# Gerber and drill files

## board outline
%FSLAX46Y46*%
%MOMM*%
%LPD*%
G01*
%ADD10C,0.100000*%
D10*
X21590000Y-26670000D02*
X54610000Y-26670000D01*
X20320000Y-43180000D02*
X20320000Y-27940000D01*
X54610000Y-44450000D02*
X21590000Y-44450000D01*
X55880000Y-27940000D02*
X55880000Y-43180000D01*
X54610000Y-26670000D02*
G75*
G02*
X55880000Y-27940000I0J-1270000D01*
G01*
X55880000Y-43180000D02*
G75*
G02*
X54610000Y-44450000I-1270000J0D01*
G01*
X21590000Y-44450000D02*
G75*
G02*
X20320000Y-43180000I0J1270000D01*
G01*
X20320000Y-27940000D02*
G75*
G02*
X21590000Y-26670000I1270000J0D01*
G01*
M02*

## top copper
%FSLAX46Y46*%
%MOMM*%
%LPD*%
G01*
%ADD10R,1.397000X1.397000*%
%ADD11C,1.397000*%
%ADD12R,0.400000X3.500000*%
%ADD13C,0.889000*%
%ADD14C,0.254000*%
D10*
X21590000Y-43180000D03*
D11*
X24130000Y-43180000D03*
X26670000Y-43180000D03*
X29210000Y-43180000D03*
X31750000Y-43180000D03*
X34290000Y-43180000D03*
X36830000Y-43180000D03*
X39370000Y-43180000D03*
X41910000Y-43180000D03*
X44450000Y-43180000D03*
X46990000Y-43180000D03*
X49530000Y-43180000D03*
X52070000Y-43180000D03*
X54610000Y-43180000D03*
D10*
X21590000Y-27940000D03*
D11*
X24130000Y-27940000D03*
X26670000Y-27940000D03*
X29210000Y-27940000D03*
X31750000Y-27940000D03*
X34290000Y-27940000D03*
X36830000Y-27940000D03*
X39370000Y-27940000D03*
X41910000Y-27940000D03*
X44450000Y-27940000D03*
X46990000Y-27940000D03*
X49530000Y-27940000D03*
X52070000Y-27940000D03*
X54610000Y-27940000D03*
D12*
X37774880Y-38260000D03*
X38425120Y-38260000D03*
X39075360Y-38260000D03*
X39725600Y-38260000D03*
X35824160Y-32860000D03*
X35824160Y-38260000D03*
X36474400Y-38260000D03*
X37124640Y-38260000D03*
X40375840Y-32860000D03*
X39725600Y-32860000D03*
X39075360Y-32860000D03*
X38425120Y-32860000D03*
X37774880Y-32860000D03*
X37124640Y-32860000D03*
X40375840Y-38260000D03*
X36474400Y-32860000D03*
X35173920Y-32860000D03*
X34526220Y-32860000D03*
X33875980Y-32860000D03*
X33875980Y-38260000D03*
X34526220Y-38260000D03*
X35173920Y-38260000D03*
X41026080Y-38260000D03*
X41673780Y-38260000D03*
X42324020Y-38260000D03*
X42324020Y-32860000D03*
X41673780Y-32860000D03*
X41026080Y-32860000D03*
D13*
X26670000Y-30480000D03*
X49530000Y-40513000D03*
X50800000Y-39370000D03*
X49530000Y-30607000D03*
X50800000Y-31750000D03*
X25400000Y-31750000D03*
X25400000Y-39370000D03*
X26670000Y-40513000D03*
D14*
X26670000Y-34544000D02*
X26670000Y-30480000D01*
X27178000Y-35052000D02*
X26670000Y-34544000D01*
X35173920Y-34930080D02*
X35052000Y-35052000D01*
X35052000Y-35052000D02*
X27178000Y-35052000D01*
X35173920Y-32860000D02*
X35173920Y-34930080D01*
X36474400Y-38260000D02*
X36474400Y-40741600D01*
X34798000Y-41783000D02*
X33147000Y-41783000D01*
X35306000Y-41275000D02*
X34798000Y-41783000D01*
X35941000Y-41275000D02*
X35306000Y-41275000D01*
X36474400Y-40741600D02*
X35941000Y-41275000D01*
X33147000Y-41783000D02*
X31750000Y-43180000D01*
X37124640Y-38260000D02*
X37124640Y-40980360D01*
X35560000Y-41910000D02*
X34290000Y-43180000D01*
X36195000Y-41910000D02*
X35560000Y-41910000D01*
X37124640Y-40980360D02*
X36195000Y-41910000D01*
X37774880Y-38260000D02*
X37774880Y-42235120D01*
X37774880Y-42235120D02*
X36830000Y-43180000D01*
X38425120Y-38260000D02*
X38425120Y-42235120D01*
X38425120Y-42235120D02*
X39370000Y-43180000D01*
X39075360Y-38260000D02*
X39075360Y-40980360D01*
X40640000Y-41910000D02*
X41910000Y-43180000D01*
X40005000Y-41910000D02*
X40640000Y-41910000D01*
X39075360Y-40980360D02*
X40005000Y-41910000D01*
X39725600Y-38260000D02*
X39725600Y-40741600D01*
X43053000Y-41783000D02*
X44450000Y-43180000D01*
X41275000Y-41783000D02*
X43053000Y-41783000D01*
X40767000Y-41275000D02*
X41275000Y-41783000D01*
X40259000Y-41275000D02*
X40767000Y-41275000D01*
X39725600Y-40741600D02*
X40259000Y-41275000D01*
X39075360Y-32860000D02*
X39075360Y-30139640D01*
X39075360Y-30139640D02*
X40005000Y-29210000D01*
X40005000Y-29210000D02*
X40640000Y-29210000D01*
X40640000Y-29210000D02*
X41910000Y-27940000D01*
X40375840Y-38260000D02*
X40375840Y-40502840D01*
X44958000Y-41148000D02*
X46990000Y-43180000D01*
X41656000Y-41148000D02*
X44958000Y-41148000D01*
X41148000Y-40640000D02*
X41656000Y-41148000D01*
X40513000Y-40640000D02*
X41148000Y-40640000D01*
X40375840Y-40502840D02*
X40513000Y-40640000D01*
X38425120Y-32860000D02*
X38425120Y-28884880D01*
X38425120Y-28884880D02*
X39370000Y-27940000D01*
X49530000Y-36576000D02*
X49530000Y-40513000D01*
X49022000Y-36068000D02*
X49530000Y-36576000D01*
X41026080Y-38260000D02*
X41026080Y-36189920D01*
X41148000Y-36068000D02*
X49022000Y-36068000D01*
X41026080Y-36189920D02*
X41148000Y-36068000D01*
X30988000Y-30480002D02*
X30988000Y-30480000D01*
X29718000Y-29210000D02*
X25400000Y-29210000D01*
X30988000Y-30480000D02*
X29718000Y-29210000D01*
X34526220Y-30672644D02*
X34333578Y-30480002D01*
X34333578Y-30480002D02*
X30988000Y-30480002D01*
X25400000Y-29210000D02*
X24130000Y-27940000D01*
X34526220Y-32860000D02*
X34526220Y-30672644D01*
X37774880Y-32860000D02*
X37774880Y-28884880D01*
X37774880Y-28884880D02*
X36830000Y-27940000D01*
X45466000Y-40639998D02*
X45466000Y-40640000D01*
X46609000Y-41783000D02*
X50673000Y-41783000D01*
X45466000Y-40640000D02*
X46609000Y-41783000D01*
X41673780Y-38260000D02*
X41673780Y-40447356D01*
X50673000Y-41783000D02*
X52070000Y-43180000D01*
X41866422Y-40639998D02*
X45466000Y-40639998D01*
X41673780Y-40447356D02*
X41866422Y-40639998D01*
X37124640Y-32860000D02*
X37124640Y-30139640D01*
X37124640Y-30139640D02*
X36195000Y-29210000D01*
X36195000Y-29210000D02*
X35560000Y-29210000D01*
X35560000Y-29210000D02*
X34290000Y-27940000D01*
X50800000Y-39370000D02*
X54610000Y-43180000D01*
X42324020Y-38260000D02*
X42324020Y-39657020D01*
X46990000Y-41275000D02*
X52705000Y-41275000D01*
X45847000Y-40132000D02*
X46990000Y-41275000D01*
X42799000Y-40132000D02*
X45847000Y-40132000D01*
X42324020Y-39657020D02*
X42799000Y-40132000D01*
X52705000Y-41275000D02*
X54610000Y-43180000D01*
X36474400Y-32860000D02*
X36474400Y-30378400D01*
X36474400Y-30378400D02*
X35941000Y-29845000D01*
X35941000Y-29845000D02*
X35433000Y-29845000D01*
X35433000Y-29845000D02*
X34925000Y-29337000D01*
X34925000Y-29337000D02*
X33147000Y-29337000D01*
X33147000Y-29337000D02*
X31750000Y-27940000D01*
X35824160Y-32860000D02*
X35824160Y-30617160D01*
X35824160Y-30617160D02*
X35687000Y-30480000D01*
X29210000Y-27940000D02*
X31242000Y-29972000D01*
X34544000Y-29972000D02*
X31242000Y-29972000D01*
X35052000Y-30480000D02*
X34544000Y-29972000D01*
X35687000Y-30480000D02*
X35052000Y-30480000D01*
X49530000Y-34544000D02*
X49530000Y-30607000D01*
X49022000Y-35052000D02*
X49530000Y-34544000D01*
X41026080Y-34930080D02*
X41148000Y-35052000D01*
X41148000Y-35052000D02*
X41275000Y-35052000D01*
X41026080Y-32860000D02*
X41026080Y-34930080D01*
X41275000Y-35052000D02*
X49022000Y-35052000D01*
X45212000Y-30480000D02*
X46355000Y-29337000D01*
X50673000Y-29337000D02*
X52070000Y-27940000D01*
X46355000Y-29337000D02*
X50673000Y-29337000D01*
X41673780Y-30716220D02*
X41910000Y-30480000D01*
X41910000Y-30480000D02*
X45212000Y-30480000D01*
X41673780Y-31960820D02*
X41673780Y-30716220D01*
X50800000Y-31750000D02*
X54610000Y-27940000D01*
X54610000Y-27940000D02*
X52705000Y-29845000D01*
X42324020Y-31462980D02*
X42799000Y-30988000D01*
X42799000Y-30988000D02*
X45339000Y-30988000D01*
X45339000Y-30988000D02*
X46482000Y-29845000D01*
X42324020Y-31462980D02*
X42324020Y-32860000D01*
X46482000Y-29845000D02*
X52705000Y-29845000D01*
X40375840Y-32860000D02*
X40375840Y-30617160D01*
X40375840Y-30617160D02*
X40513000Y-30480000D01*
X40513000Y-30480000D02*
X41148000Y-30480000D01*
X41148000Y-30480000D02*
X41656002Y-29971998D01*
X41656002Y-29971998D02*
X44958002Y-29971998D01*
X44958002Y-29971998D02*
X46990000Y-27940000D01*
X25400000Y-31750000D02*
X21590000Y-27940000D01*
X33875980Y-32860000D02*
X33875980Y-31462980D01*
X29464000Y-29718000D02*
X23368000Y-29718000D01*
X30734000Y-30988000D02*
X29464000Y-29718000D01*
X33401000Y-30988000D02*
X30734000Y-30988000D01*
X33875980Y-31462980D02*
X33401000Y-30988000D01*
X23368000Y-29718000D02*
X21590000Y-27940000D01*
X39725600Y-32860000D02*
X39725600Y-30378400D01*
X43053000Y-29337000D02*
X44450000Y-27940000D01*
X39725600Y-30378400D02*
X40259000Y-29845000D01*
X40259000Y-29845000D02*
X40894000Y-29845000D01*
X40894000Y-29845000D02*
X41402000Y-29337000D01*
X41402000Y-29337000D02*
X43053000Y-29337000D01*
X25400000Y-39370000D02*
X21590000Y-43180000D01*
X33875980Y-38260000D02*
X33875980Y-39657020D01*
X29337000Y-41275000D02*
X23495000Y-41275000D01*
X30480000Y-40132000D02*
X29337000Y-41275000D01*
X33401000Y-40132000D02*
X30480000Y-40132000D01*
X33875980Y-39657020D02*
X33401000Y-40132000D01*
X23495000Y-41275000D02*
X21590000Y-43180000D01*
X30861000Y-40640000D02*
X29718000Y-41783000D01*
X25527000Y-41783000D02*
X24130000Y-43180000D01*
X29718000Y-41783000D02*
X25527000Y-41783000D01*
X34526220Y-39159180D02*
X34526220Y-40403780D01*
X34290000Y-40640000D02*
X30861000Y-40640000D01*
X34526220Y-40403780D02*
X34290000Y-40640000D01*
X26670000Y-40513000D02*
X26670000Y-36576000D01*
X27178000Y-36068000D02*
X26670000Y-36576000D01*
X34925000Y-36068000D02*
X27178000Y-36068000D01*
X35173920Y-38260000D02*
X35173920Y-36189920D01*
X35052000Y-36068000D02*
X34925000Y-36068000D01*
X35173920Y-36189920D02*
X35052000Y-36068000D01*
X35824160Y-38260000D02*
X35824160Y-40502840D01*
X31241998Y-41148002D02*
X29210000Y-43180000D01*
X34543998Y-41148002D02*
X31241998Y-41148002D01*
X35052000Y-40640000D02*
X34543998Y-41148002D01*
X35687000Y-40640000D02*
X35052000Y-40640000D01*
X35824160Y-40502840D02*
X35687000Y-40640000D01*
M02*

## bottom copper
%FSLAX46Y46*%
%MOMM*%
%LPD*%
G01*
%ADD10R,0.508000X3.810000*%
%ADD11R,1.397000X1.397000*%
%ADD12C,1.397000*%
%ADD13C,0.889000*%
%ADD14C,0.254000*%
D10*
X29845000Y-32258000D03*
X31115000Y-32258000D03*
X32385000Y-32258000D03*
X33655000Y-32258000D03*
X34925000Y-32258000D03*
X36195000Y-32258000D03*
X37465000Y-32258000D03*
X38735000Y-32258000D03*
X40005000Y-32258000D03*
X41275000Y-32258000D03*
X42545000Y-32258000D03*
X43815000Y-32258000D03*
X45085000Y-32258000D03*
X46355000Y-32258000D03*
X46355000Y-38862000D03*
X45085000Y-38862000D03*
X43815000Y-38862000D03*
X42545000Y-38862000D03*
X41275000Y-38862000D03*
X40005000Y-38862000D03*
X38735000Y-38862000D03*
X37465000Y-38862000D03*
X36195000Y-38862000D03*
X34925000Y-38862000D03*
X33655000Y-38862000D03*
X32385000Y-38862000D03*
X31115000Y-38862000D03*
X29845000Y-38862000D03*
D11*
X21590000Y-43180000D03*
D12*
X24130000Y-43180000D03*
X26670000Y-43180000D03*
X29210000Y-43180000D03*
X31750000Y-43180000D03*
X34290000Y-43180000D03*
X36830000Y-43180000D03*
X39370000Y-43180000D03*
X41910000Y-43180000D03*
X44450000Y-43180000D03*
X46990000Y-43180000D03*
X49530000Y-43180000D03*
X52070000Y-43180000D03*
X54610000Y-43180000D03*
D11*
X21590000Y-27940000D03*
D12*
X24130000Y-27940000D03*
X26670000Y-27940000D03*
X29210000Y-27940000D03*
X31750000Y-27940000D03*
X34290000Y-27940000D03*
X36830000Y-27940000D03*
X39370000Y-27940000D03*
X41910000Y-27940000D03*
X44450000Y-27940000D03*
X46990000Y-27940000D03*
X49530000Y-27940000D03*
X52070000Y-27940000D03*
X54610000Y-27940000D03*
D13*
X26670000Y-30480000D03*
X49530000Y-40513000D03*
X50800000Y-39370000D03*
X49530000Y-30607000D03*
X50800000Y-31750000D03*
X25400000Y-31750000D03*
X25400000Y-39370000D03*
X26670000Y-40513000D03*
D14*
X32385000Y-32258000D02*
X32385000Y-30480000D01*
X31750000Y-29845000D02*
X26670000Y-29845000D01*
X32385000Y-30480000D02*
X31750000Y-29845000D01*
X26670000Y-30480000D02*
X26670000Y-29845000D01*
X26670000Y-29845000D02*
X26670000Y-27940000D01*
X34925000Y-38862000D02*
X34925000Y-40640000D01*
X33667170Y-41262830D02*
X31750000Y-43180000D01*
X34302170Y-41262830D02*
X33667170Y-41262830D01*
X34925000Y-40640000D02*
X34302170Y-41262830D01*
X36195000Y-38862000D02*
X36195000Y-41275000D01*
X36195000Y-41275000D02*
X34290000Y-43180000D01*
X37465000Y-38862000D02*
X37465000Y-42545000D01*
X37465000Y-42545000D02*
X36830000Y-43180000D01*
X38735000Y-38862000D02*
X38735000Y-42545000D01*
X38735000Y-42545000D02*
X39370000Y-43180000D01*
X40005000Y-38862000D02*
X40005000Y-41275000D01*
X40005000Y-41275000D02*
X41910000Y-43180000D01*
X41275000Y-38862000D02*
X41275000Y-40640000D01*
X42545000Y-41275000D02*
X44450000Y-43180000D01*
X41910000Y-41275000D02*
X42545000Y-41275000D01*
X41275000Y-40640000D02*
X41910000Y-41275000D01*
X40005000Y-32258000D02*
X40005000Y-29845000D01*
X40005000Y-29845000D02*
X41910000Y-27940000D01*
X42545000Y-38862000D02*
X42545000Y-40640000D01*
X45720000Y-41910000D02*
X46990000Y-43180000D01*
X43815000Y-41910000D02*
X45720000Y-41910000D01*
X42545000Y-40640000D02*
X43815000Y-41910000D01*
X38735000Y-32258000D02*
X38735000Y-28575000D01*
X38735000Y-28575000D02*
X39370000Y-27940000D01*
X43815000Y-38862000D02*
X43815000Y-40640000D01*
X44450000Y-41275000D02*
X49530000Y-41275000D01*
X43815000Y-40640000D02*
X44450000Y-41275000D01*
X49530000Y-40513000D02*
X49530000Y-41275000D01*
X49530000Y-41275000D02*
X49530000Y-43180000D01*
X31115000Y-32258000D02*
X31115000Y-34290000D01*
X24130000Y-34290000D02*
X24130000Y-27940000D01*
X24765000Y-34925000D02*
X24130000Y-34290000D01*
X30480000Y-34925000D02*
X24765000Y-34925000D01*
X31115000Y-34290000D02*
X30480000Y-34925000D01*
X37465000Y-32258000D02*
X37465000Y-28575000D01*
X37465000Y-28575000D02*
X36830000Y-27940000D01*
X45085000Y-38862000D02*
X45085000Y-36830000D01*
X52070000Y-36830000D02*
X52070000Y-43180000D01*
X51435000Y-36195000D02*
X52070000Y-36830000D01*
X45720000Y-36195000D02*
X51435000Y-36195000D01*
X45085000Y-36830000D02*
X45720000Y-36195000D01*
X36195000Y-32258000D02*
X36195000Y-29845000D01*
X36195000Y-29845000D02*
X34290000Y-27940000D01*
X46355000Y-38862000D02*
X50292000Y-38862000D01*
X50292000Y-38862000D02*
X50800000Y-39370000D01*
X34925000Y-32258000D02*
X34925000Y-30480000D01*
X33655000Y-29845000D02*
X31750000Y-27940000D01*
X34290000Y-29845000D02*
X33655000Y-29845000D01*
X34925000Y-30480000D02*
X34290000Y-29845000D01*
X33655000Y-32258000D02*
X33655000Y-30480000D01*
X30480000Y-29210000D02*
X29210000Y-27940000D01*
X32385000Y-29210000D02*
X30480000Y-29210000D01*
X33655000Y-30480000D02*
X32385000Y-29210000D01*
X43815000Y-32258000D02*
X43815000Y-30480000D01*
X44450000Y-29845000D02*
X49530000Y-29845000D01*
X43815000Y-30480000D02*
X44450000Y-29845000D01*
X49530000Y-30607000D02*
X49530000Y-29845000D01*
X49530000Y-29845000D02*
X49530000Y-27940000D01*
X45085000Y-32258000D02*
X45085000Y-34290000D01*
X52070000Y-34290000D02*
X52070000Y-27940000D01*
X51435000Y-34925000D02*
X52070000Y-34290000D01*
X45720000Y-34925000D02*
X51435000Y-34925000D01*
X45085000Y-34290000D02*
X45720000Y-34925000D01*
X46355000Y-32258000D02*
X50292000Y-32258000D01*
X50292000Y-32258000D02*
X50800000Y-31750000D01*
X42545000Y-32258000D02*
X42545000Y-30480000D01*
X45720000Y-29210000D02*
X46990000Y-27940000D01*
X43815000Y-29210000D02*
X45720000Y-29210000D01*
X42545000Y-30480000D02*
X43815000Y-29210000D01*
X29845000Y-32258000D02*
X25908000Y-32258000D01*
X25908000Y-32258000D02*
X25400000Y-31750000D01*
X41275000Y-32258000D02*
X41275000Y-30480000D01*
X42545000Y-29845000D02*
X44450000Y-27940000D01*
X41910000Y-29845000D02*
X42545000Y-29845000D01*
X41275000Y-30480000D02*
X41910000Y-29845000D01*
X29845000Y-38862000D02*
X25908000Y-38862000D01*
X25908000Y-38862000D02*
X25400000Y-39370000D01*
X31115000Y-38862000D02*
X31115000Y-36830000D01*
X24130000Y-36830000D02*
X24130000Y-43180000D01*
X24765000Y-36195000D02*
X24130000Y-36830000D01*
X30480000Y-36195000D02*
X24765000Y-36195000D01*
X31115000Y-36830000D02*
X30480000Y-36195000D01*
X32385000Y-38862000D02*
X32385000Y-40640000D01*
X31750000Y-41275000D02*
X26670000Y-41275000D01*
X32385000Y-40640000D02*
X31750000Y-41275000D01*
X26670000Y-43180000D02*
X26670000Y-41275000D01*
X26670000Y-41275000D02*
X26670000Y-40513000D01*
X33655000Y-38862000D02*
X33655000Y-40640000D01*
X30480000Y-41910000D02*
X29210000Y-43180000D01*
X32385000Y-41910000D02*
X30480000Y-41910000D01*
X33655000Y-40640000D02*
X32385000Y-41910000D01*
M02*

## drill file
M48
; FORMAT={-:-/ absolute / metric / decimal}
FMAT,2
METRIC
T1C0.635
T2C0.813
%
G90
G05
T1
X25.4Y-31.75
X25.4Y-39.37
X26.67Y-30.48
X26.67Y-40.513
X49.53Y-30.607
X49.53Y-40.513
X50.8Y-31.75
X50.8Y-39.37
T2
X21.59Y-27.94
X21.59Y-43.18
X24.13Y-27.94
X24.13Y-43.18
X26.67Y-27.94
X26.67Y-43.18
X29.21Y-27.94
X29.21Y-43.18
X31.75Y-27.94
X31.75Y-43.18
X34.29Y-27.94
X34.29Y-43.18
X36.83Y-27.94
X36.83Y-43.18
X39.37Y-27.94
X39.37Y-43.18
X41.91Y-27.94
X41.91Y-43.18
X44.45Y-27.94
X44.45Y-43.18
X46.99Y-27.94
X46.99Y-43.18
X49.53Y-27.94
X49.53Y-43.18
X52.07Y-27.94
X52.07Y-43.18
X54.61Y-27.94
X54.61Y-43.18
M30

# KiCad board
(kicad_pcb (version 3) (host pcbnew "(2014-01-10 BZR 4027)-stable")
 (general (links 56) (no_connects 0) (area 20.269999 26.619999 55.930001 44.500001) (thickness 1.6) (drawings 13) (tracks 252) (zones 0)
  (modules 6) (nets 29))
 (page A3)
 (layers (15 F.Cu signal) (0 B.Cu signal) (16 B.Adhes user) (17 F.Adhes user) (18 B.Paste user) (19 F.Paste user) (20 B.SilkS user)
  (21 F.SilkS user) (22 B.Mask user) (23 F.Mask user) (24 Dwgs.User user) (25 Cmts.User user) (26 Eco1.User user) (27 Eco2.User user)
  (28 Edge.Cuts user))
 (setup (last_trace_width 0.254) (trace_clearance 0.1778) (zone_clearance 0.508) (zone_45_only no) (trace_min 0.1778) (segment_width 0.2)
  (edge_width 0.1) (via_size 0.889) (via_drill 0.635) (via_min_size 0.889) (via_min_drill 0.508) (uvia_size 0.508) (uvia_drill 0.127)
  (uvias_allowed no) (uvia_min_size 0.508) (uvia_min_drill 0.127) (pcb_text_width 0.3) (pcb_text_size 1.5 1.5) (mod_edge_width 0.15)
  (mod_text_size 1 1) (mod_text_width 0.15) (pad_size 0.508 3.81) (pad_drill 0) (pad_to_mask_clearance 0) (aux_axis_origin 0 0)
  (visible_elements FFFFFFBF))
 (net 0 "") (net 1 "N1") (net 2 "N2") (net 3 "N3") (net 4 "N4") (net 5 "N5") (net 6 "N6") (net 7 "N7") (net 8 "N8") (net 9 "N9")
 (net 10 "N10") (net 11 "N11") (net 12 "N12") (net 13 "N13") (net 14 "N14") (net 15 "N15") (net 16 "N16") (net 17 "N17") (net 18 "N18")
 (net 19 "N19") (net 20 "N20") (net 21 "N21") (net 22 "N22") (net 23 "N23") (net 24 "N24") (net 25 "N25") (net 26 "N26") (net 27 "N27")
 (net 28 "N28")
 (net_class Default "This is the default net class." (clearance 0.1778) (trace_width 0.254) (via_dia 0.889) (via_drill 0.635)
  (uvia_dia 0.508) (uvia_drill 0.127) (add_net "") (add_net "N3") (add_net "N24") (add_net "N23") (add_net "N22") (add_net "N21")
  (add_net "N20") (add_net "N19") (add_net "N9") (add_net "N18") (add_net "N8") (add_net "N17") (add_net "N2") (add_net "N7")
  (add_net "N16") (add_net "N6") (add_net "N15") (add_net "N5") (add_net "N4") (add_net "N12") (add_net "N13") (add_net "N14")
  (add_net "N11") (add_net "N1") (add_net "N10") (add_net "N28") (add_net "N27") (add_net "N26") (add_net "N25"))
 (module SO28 (layer B.Cu) (at 38.1 35.56)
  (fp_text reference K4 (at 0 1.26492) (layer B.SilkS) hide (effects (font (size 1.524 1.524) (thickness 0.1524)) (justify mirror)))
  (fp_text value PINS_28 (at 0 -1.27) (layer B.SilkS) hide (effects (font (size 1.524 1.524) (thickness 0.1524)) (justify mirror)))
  (pad 1 smd rect (at -8.255 -3.302) (size 0.508 3.81) (layers B.Cu B.Paste B.Mask) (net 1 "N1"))
  (pad 2 smd rect (at -6.985 -3.302) (size 0.508 3.81) (layers B.Cu B.Paste B.Mask) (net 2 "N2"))
  (pad 3 smd rect (at -5.715 -3.302) (size 0.508 3.81) (layers B.Cu B.Paste B.Mask) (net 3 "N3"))
  (pad 4 smd rect (at -4.445 -3.302) (size 0.508 3.81) (layers B.Cu B.Paste B.Mask) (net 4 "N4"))
  (pad 5 smd rect (at -3.175 -3.302) (size 0.508 3.81) (layers B.Cu B.Paste B.Mask) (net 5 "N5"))
  (pad 6 smd rect (at -1.905 -3.302) (size 0.508 3.81) (layers B.Cu B.Paste B.Mask) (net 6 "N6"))
  (pad 7 smd rect (at -0.635 -3.302) (size 0.508 3.81) (layers B.Cu B.Paste B.Mask) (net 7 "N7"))
  (pad 8 smd rect (at 0.635 -3.302) (size 0.508 3.81) (layers B.Cu B.Paste B.Mask) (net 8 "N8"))
  (pad 9 smd rect (at 1.905 -3.302) (size 0.508 3.81) (layers B.Cu B.Paste B.Mask) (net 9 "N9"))
  (pad 10 smd rect (at 3.175 -3.302) (size 0.508 3.81) (layers B.Cu B.Paste B.Mask) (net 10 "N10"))
  (pad 11 smd rect (at 4.445 -3.302) (size 0.508 3.81) (layers B.Cu B.Paste B.Mask) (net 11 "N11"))
  (pad 12 smd rect (at 5.715 -3.302) (size 0.508 3.81) (layers B.Cu B.Paste B.Mask) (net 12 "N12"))
  (pad 13 smd rect (at 6.985 -3.302) (size 0.508 3.81) (layers B.Cu B.Paste B.Mask) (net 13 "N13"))
  (pad 14 smd rect (at 8.255 -3.302) (size 0.508 3.81) (layers B.Cu B.Paste B.Mask) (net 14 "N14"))
  (pad 15 smd rect (at 8.255 3.302) (size 0.508 3.81) (layers B.Cu B.Paste B.Mask) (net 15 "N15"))
  (pad 16 smd rect (at 6.985 3.302) (size 0.508 3.81) (layers B.Cu B.Paste B.Mask) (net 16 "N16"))
  (pad 17 smd rect (at 5.715 3.302) (size 0.508 3.81) (layers B.Cu B.Paste B.Mask) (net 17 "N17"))
  (pad 18 smd rect (at 4.445 3.302) (size 0.508 3.81) (layers B.Cu B.Paste B.Mask) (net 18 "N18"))
  (pad 19 smd rect (at 3.175 3.302) (size 0.508 3.81) (layers B.Cu B.Paste B.Mask) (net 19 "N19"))
  (pad 20 smd rect (at 1.905 3.302) (size 0.508 3.81) (layers B.Cu B.Paste B.Mask) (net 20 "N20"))
  (pad 21 smd rect (at 0.635 3.302) (size 0.508 3.81) (layers B.Cu B.Paste B.Mask) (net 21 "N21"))
  (pad 22 smd rect (at -0.635 3.302) (size 0.508 3.81) (layers B.Cu B.Paste B.Mask) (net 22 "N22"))
  (pad 23 smd rect (at -1.905 3.302) (size 0.508 3.81) (layers B.Cu B.Paste B.Mask) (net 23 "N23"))
  (pad 24 smd rect (at -3.175 3.302) (size 0.508 3.81) (layers B.Cu B.Paste B.Mask) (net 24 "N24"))
  (pad 25 smd rect (at -4.445 3.302) (size 0.508 3.81) (layers B.Cu B.Paste B.Mask) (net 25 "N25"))
  (pad 26 smd rect (at -5.715 3.302) (size 0.508 3.81) (layers B.Cu B.Paste B.Mask) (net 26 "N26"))
  (pad 27 smd rect (at -6.985 3.302) (size 0.508 3.81) (layers B.Cu B.Paste B.Mask) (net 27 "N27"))
  (pad 28 smd rect (at -8.255 3.302) (size 0.508 3.81) (layers B.Cu B.Paste B.Mask) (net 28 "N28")))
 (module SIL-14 (layer F.Cu) (at 38.1 43.18)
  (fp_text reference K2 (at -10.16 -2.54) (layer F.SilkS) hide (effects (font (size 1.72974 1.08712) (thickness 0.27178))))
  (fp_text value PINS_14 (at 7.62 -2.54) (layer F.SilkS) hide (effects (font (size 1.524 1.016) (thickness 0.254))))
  (pad 1 thru_hole rect (at -16.51 0) (size 1.397 1.397) (drill 0.8128) (layers *.Cu *.Mask F.SilkS) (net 28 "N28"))
  (pad 2 thru_hole circle (at -13.97 0) (size 1.397 1.397) (drill 0.8128) (layers *.Cu *.Mask F.SilkS) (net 27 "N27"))
  (pad 3 thru_hole circle (at -11.43 0) (size 1.397 1.397) (drill 0.8128) (layers *.Cu *.Mask F.SilkS) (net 26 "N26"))
  (pad 4 thru_hole circle (at -8.89 0) (size 1.397 1.397) (drill 0.8128) (layers *.Cu *.Mask F.SilkS) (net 25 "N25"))
  (pad 5 thru_hole circle (at -6.35 0) (size 1.397 1.397) (drill 0.8128) (layers *.Cu *.Mask F.SilkS) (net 24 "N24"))
  (pad 6 thru_hole circle (at -3.81 0) (size 1.397 1.397) (drill 0.8128) (layers *.Cu *.Mask F.SilkS) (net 23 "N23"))
  (pad 7 thru_hole circle (at -1.27 0) (size 1.397 1.397) (drill 0.8128) (layers *.Cu *.Mask F.SilkS) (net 22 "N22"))
  (pad 8 thru_hole circle (at 1.27 0) (size 1.397 1.397) (drill 0.8128) (layers *.Cu *.Mask F.SilkS) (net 21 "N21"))
  (pad 9 thru_hole circle (at 3.81 0) (size 1.397 1.397) (drill 0.8128) (layers *.Cu *.Mask F.SilkS) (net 20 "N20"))
  (pad 10 thru_hole circle (at 6.35 0) (size 1.397 1.397) (drill 0.8128) (layers *.Cu *.Mask F.SilkS) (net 19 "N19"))
  (pad 11 thru_hole circle (at 8.89 0) (size 1.397 1.397) (drill 0.8128) (layers *.Cu *.Mask F.SilkS) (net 18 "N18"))
  (pad 12 thru_hole circle (at 11.43 0) (size 1.397 1.397) (drill 0.8128) (layers *.Cu *.Mask F.SilkS) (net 17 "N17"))
  (pad 13 thru_hole circle (at 13.97 0) (size 1.397 1.397) (drill 0.8128) (layers *.Cu *.Mask F.SilkS) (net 16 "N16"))
  (pad 14 thru_hole circle (at 16.51 0) (size 1.397 1.397) (drill 0.8128) (layers *.Cu *.Mask F.SilkS) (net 15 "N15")))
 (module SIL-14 (layer F.Cu) (at 38.1 27.94)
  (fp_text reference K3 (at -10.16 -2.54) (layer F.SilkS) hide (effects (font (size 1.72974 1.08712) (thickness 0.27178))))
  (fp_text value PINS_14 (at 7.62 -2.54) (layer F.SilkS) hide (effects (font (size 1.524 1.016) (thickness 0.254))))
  (pad 1 thru_hole rect (at -16.51 0) (size 1.397 1.397) (drill 0.8128) (layers *.Cu *.Mask F.SilkS) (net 1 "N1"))
  (pad 2 thru_hole circle (at -13.97 0) (size 1.397 1.397) (drill 0.8128) (layers *.Cu *.Mask F.SilkS) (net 2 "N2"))
  (pad 3 thru_hole circle (at -11.43 0) (size 1.397 1.397) (drill 0.8128) (layers *.Cu *.Mask F.SilkS) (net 3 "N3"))
  (pad 4 thru_hole circle (at -8.89 0) (size 1.397 1.397) (drill 0.8128) (layers *.Cu *.Mask F.SilkS) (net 4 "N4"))
  (pad 5 thru_hole circle (at -6.35 0) (size 1.397 1.397) (drill 0.8128) (layers *.Cu *.Mask F.SilkS) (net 5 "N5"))
  (pad 6 thru_hole circle (at -3.81 0) (size 1.397 1.397) (drill 0.8128) (layers *.Cu *.Mask F.SilkS) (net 6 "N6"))
  (pad 7 thru_hole circle (at -1.27 0) (size 1.397 1.397) (drill 0.8128) (layers *.Cu *.Mask F.SilkS) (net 7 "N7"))
  (pad 8 thru_hole circle (at 1.27 0) (size 1.397 1.397) (drill 0.8128) (layers *.Cu *.Mask F.SilkS) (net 8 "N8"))
  (pad 9 thru_hole circle (at 3.81 0) (size 1.397 1.397) (drill 0.8128) (layers *.Cu *.Mask F.SilkS) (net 9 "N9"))
  (pad 10 thru_hole circle (at 6.35 0) (size 1.397 1.397) (drill 0.8128) (layers *.Cu *.Mask F.SilkS) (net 10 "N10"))
  (pad 11 thru_hole circle (at 8.89 0) (size 1.397 1.397) (drill 0.8128) (layers *.Cu *.Mask F.SilkS) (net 11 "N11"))
  (pad 12 thru_hole circle (at 11.43 0) (size 1.397 1.397) (drill 0.8128) (layers *.Cu *.Mask F.SilkS) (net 12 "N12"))
  (pad 13 thru_hole circle (at 13.97 0) (size 1.397 1.397) (drill 0.8128) (layers *.Cu *.Mask F.SilkS) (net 13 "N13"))
  (pad 14 thru_hole circle (at 16.51 0) (size 1.397 1.397) (drill 0.8128) (layers *.Cu *.Mask F.SilkS) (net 14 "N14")))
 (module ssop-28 (layer F.Cu) (at 38.1 35.56)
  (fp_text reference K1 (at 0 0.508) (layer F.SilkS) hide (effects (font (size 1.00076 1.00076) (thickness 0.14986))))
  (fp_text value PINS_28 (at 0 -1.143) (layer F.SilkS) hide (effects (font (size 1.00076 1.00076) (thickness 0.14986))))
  (pad 7 smd rect (at -0.32512 2.7) (size 0.4 3.5) (layers F.Cu F.Paste F.Mask) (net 22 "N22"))
  (pad 8 smd rect (at 0.32512 2.7) (size 0.4 3.5) (layers F.Cu F.Paste F.Mask) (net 21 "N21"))
  (pad 9 smd rect (at 0.97536 2.7) (size 0.4 3.5) (layers F.Cu F.Paste F.Mask) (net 20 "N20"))
  (pad 10 smd rect (at 1.6256 2.7) (size 0.4 3.5) (layers F.Cu F.Paste F.Mask) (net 19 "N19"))
  (pad 25 smd rect (at -2.27584 -2.7) (size 0.4 3.5) (layers F.Cu F.Paste F.Mask) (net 4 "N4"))
  (pad 4 smd rect (at -2.27584 2.7) (size 0.4 3.5) (layers F.Cu F.Paste F.Mask) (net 25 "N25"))
  (pad 5 smd rect (at -1.6256 2.7) (size 0.4 3.5) (layers F.Cu F.Paste F.Mask) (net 24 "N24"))
  (pad 6 smd rect (at -0.97536 2.7) (size 0.4 3.5) (layers F.Cu F.Paste F.Mask) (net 23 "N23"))
  (pad 18 smd rect (at 2.27584 -2.7) (size 0.4 3.5) (layers F.Cu F.Paste F.Mask) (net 11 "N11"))
  (pad 19 smd rect (at 1.6256 -2.7) (size 0.4 3.5) (layers F.Cu F.Paste F.Mask) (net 10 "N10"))
  (pad 20 smd rect (at 0.97536 -2.7) (size 0.4 3.5) (layers F.Cu F.Paste F.Mask) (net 9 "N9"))
  (pad 21 smd rect (at 0.32512 -2.7) (size 0.4 3.5) (layers F.Cu F.Paste F.Mask) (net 8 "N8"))
  (pad 22 smd rect (at -0.32512 -2.7) (size 0.4 3.5) (layers F.Cu F.Paste F.Mask) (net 7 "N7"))
  (pad 23 smd rect (at -0.97536 -2.7) (size 0.4 3.5) (layers F.Cu F.Paste F.Mask) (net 6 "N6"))
  (pad 11 smd rect (at 2.27584 2.7) (size 0.4 3.5) (layers F.Cu F.Paste F.Mask) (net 18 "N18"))
  (pad 24 smd rect (at -1.6256 -2.7) (size 0.4 3.5) (layers F.Cu F.Paste F.Mask) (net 5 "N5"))
  (pad 26 smd rect (at -2.92608 -2.7) (size 0.4 3.5) (layers F.Cu F.Paste F.Mask) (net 3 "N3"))
  (pad 27 smd rect (at -3.57378 -2.7) (size 0.4 3.5) (layers F.Cu F.Paste F.Mask) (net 2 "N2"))
  (pad 28 smd rect (at -4.22402 -2.7) (size 0.4 3.5) (layers F.Cu F.Paste F.Mask) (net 1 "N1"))
  (pad 1 smd rect (at -4.22402 2.7) (size 0.4 3.5) (layers F.Cu F.Paste F.Mask) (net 28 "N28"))
  (pad 2 smd rect (at -3.57378 2.7) (size 0.4 3.5) (layers F.Cu F.Paste F.Mask) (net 27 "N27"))
  (pad 3 smd rect (at -2.92608 2.7) (size 0.4 3.5) (layers F.Cu F.Paste F.Mask) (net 26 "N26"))
  (pad 12 smd rect (at 2.92608 2.7) (size 0.4 3.5) (layers F.Cu F.Paste F.Mask) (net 17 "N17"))
  (pad 13 smd rect (at 3.57378 2.7) (size 0.4 3.5) (layers F.Cu F.Paste F.Mask) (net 16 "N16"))
  (pad 14 smd rect (at 4.22402 2.7) (size 0.4 3.5) (layers F.Cu F.Paste F.Mask) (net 15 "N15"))
  (pad 15 smd rect (at 4.22402 -2.7) (size 0.4 3.5) (layers F.Cu F.Paste F.Mask) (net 14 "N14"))
  (pad 16 smd rect (at 3.57378 -2.7) (size 0.4 3.5) (layers F.Cu F.Paste F.Mask) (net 13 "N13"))
  (pad 17 smd rect (at 2.92608 -2.7) (size 0.4 3.5) (layers F.Cu F.Paste F.Mask) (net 12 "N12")))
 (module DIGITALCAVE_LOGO (layer F.Cu) (at 23.495 35.56)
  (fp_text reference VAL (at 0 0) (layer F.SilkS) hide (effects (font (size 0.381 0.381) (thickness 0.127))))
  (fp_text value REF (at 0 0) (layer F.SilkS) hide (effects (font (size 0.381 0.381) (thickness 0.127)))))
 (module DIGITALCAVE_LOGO (layer B.Cu) (at 23.495 35.56)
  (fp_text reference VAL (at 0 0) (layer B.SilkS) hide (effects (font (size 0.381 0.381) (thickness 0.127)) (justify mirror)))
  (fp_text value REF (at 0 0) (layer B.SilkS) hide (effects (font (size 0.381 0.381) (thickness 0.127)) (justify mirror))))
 (gr_line (start 21.59 26.67) (end 54.61 26.67) (angle 90) (layer Edge.Cuts) (width 0.1))
 (gr_line (start 20.32 43.18) (end 20.32 27.94) (angle 90) (layer Edge.Cuts) (width 0.1))
 (gr_line (start 54.61 44.45) (end 21.59 44.45) (angle 90) (layer Edge.Cuts) (width 0.1))
 (gr_line (start 55.88 27.94) (end 55.88 43.18) (angle 90) (layer Edge.Cuts) (width 0.1))
 (gr_arc (start 54.61 27.94) (end 54.61 26.67) (angle 90) (layer Edge.Cuts) (width 0.1))
 (gr_arc (start 54.61 43.18) (end 55.88 43.18) (angle 90) (layer Edge.Cuts) (width 0.1))
 (gr_arc (start 21.59 43.18) (end 21.59 44.45) (angle 90) (layer Edge.Cuts) (width 0.1))
 (gr_arc (start 21.59 27.94) (end 20.32 27.94) (angle 90) (layer Edge.Cuts) (width 0.1))
 (segment (start 32.385 32.258) (end 32.385 30.48) (width 0.254) (layer B.Cu) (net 3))
 (segment (start 31.75 29.845) (end 26.67 29.845) (width 0.254) (layer B.Cu) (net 3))
 (segment (start 32.385 30.48) (end 31.75 29.845) (width 0.254) (layer B.Cu) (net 3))
 (segment (start 26.67 34.544) (end 26.67 30.48) (width 0.254) (layer F.Cu) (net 3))
 (via (at 26.67 30.48) (size 0.889) (layers F.Cu B.Cu) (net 3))
 (segment (start 27.178 35.052) (end 26.67 34.544) (width 0.254) (layer F.Cu) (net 3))
 (segment (start 35.17392 34.93008) (end 35.052 35.052) (width 0.254) (layer F.Cu) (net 3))
 (segment (start 35.052 35.052) (end 27.178 35.052) (width 0.254) (layer F.Cu) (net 3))
 (segment (start 26.67 30.48) (end 26.67 29.845) (width 0.254) (layer B.Cu) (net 3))
 (segment (start 26.67 29.845) (end 26.67 27.94) (width 0.254) (layer B.Cu) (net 3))
 (segment (start 35.17392 32.86) (end 35.17392 34.93008) (width 0.254) (layer F.Cu) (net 3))
 (segment (start 34.925 38.862) (end 34.925 40.64) (width 0.254) (layer B.Cu) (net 24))
 (segment (start 33.66717 41.26283) (end 31.75 43.18) (width 0.254) (layer B.Cu) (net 24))
 (segment (start 34.30217 41.26283) (end 33.66717 41.26283) (width 0.254) (layer B.Cu) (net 24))
 (segment (start 34.925 40.64) (end 34.30217 41.26283) (width 0.254) (layer B.Cu) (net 24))
 (segment (start 36.4744 38.26) (end 36.4744 40.7416) (width 0.254) (layer F.Cu) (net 24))
 (segment (start 34.798 41.783) (end 33.147 41.783) (width 0.254) (layer F.Cu) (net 24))
 (segment (start 35.306 41.275) (end 34.798 41.783) (width 0.254) (layer F.Cu) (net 24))
 (segment (start 35.941 41.275) (end 35.306 41.275) (width 0.254) (layer F.Cu) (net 24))
 (segment (start 36.4744 40.7416) (end 35.941 41.275) (width 0.254) (layer F.Cu) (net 24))
 (segment (start 33.147 41.783) (end 31.75 43.18) (width 0.254) (layer F.Cu) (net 24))
 (segment (start 36.195 38.862) (end 36.195 41.275) (width 0.254) (layer B.Cu) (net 23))
 (segment (start 36.195 41.275) (end 34.29 43.18) (width 0.254) (layer B.Cu) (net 23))
 (segment (start 37.12464 38.26) (end 37.12464 40.98036) (width 0.254) (layer F.Cu) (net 23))
 (segment (start 35.56 41.91) (end 34.29 43.18) (width 0.254) (layer F.Cu) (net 23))
 (segment (start 36.195 41.91) (end 35.56 41.91) (width 0.254) (layer F.Cu) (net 23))
 (segment (start 37.12464 40.98036) (end 36.195 41.91) (width 0.254) (layer F.Cu) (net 23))
 (segment (start 37.465 38.862) (end 37.465 42.545) (width 0.254) (layer B.Cu) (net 22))
 (segment (start 37.465 42.545) (end 36.83 43.18) (width 0.254) (layer B.Cu) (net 22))
 (segment (start 37.77488 38.26) (end 37.77488 42.23512) (width 0.254) (layer F.Cu) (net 22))
 (segment (start 37.77488 42.23512) (end 36.83 43.18) (width 0.254) (layer F.Cu) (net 22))
 (segment (start 38.735 38.862) (end 38.735 42.545) (width 0.254) (layer B.Cu) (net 21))
 (segment (start 38.735 42.545) (end 39.37 43.18) (width 0.254) (layer B.Cu) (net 21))
 (segment (start 38.42512 38.26) (end 38.42512 42.23512) (width 0.254) (layer F.Cu) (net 21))
 (segment (start 38.42512 42.23512) (end 39.37 43.18) (width 0.254) (layer F.Cu) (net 21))
 (segment (start 40.005 38.862) (end 40.005 41.275) (width 0.254) (layer B.Cu) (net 20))
 (segment (start 40.005 41.275) (end 41.91 43.18) (width 0.254) (layer B.Cu) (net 20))
 (segment (start 39.07536 38.26) (end 39.07536 40.98036) (width 0.254) (layer F.Cu) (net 20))
 (segment (start 40.64 41.91) (end 41.91 43.18) (width 0.254) (layer F.Cu) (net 20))
 (segment (start 40.005 41.91) (end 40.64 41.91) (width 0.254) (layer F.Cu) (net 20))
 (segment (start 39.07536 40.98036) (end 40.005 41.91) (width 0.254) (layer F.Cu) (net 20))
 (segment (start 41.275 38.862) (end 41.275 40.64) (width 0.254) (layer B.Cu) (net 19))
 (segment (start 42.545 41.275) (end 44.45 43.18) (width 0.254) (layer B.Cu) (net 19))
 (segment (start 41.91 41.275) (end 42.545 41.275) (width 0.254) (layer B.Cu) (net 19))
 (segment (start 41.275 40.64) (end 41.91 41.275) (width 0.254) (layer B.Cu) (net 19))
 (segment (start 39.7256 38.26) (end 39.7256 40.7416) (width 0.254) (layer F.Cu) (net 19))
 (segment (start 43.053 41.783) (end 44.45 43.18) (width 0.254) (layer F.Cu) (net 19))
 (segment (start 41.275 41.783) (end 43.053 41.783) (width 0.254) (layer F.Cu) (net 19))
 (segment (start 40.767 41.275) (end 41.275 41.783) (width 0.254) (layer F.Cu) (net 19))
 (segment (start 40.259 41.275) (end 40.767 41.275) (width 0.254) (layer F.Cu) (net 19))
 (segment (start 39.7256 40.7416) (end 40.259 41.275) (width 0.254) (layer F.Cu) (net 19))
 (segment (start 40.005 32.258) (end 40.005 29.845) (width 0.254) (layer B.Cu) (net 9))
 (segment (start 40.005 29.845) (end 41.91 27.94) (width 0.254) (layer B.Cu) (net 9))
 (segment (start 39.07536 32.86) (end 39.07536 30.13964) (width 0.254) (layer F.Cu) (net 9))
 (segment (start 39.07536 30.13964) (end 40.005 29.21) (width 0.254) (layer F.Cu) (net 9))
 (segment (start 40.005 29.21) (end 40.64 29.21) (width 0.254) (layer F.Cu) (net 9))
 (segment (start 40.64 29.21) (end 41.91 27.94) (width 0.254) (layer F.Cu) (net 9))
 (segment (start 42.545 38.862) (end 42.545 40.64) (width 0.254) (layer B.Cu) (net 18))
 (segment (start 45.72 41.91) (end 46.99 43.18) (width 0.254) (layer B.Cu) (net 18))
 (segment (start 43.815 41.91) (end 45.72 41.91) (width 0.254) (layer B.Cu) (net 18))
 (segment (start 42.545 40.64) (end 43.815 41.91) (width 0.254) (layer B.Cu) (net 18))
 (segment (start 40.37584 38.26) (end 40.37584 40.50284) (width 0.254) (layer F.Cu) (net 18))
 (segment (start 44.958 41.148) (end 46.99 43.18) (width 0.254) (layer F.Cu) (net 18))
 (segment (start 41.656 41.148) (end 44.958 41.148) (width 0.254) (layer F.Cu) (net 18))
 (segment (start 41.148 40.64) (end 41.656 41.148) (width 0.254) (layer F.Cu) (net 18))
 (segment (start 40.513 40.64) (end 41.148 40.64) (width 0.254) (layer F.Cu) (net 18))
 (segment (start 40.37584 40.50284) (end 40.513 40.64) (width 0.254) (layer F.Cu) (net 18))
 (segment (start 38.735 32.258) (end 38.735 28.575) (width 0.254) (layer B.Cu) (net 8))
 (segment (start 38.735 28.575) (end 39.37 27.94) (width 0.254) (layer B.Cu) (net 8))
 (segment (start 38.42512 32.86) (end 38.42512 28.88488) (width 0.254) (layer F.Cu) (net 8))
 (segment (start 38.42512 28.88488) (end 39.37 27.94) (width 0.254) (layer F.Cu) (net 8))
 (segment (start 43.815 38.862) (end 43.815 40.64) (width 0.254) (layer B.Cu) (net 17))
 (segment (start 44.45 41.275) (end 49.53 41.275) (width 0.254) (layer B.Cu) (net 17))
 (segment (start 43.815 40.64) (end 44.45 41.275) (width 0.254) (layer B.Cu) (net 17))
 (segment (start 49.53 36.576) (end 49.53 40.513) (width 0.254) (layer F.Cu) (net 17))
 (via (at 49.53 40.513) (size 0.889) (layers F.Cu B.Cu) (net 17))
 (segment (start 49.022 36.068) (end 49.53 36.576) (width 0.254) (layer F.Cu) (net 17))
 (segment (start 41.02608 38.26) (end 41.02608 36.18992) (width 0.254) (layer F.Cu) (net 17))
 (segment (start 49.53 40.513) (end 49.53 41.275) (width 0.254) (layer B.Cu) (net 17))
 (segment (start 49.53 41.275) (end 49.53 43.18) (width 0.254) (layer B.Cu) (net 17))
 (segment (start 41.148 36.068) (end 49.022 36.068) (width 0.254) (layer F.Cu) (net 17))
 (segment (start 41.02608 36.18992) (end 41.148 36.068) (width 0.254) (layer F.Cu) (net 17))
 (segment (start 31.115 32.258) (end 31.115 34.29) (width 0.254) (layer B.Cu) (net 2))
 (segment (start 24.13 34.29) (end 24.13 27.94) (width 0.254) (layer B.Cu) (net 2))
 (segment (start 24.765 34.925) (end 24.13 34.29) (width 0.254) (layer B.Cu) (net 2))
 (segment (start 30.48 34.925) (end 24.765 34.925) (width 0.254) (layer B.Cu) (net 2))
 (segment (start 31.115 34.29) (end 30.48 34.925) (width 0.254) (layer B.Cu) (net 2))
 (segment (start 30.988 30.480002) (end 30.988 30.48) (width 0.254) (layer F.Cu) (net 2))
 (segment (start 29.718 29.21) (end 25.4 29.21) (width 0.254) (layer F.Cu) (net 2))
 (segment (start 30.988 30.48) (end 29.718 29.21) (width 0.254) (layer F.Cu) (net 2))
 (segment (start 34.52622 30.672644) (end 34.333578 30.480002) (width 0.254) (layer F.Cu) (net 2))
 (segment (start 34.333578 30.480002) (end 30.988 30.480002) (width 0.254) (layer F.Cu) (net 2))
 (segment (start 25.4 29.21) (end 24.13 27.94) (width 0.254) (layer F.Cu) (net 2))
 (segment (start 34.52622 32.86) (end 34.52622 30.672644) (width 0.254) (layer F.Cu) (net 2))
 (segment (start 37.465 32.258) (end 37.465 28.575) (width 0.254) (layer B.Cu) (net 7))
 (segment (start 37.465 28.575) (end 36.83 27.94) (width 0.254) (layer B.Cu) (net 7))
 (segment (start 37.77488 32.86) (end 37.77488 28.88488) (width 0.254) (layer F.Cu) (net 7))
 (segment (start 37.77488 28.88488) (end 36.83 27.94) (width 0.254) (layer F.Cu) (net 7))
 (segment (start 45.085 38.862) (end 45.085 36.83) (width 0.254) (layer B.Cu) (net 16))
 (segment (start 52.07 36.83) (end 52.07 43.18) (width 0.254) (layer B.Cu) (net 16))
 (segment (start 51.435 36.195) (end 52.07 36.83) (width 0.254) (layer B.Cu) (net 16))
 (segment (start 45.72 36.195) (end 51.435 36.195) (width 0.254) (layer B.Cu) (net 16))
 (segment (start 45.085 36.83) (end 45.72 36.195) (width 0.254) (layer B.Cu) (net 16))
 (segment (start 45.466 40.639998) (end 45.466 40.64) (width 0.254) (layer F.Cu) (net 16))
 (segment (start 46.609 41.783) (end 50.673 41.783) (width 0.254) (layer F.Cu) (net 16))
 (segment (start 45.466 40.64) (end 46.609 41.783) (width 0.254) (layer F.Cu) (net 16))
 (segment (start 41.67378 38.26) (end 41.67378 40.447356) (width 0.254) (layer F.Cu) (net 16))
 (segment (start 50.673 41.783) (end 52.07 43.18) (width 0.254) (layer F.Cu) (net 16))
 (segment (start 41.866422 40.639998) (end 45.466 40.639998) (width 0.254) (layer F.Cu) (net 16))
 (segment (start 41.67378 40.447356) (end 41.866422 40.639998) (width 0.254) (layer F.Cu) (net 16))
 (segment (start 36.195 32.258) (end 36.195 29.845) (width 0.254) (layer B.Cu) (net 6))
 (segment (start 36.195 29.845) (end 34.29 27.94) (width 0.254) (layer B.Cu) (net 6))
 (segment (start 37.12464 32.86) (end 37.12464 30.13964) (width 0.254) (layer F.Cu) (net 6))
 (segment (start 37.12464 30.13964) (end 36.195 29.21) (width 0.254) (layer F.Cu) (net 6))
 (segment (start 36.195 29.21) (end 35.56 29.21) (width 0.254) (layer F.Cu) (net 6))
 (segment (start 35.56 29.21) (end 34.29 27.94) (width 0.254) (layer F.Cu) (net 6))
 (segment (start 46.355 38.862) (end 50.292 38.862) (width 0.254) (layer B.Cu) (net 15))
 (segment (start 50.8 39.37) (end 54.61 43.18) (width 0.254) (layer F.Cu) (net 15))
 (via (at 50.8 39.37) (size 0.889) (layers F.Cu B.Cu) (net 15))
 (segment (start 50.292 38.862) (end 50.8 39.37) (width 0.254) (layer B.Cu) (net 15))
 (segment (start 42.32402 38.26) (end 42.32402 39.65702) (width 0.254) (layer F.Cu) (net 15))
 (segment (start 46.99 41.275) (end 52.705 41.275) (width 0.254) (layer F.Cu) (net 15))
 (segment (start 45.847 40.132) (end 46.99 41.275) (width 0.254) (layer F.Cu) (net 15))
 (segment (start 42.799 40.132) (end 45.847 40.132) (width 0.254) (layer F.Cu) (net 15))
 (segment (start 42.32402 39.65702) (end 42.799 40.132) (width 0.254) (layer F.Cu) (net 15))
 (segment (start 52.705 41.275) (end 54.61 43.18) (width 0.254) (layer F.Cu) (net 15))
 (segment (start 34.925 32.258) (end 34.925 30.48) (width 0.254) (layer B.Cu) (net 5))
 (segment (start 33.655 29.845) (end 31.75 27.94) (width 0.254) (layer B.Cu) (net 5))
 (segment (start 34.29 29.845) (end 33.655 29.845) (width 0.254) (layer B.Cu) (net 5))
 (segment (start 34.925 30.48) (end 34.29 29.845) (width 0.254) (layer B.Cu) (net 5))
 (segment (start 36.4744 32.86) (end 36.4744 30.3784) (width 0.254) (layer F.Cu) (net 5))
 (segment (start 36.4744 30.3784) (end 35.941 29.845) (width 0.254) (layer F.Cu) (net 5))
 (segment (start 35.941 29.845) (end 35.433 29.845) (width 0.254) (layer F.Cu) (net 5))
 (segment (start 35.433 29.845) (end 34.925 29.337) (width 0.254) (layer F.Cu) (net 5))
 (segment (start 34.925 29.337) (end 33.147 29.337) (width 0.254) (layer F.Cu) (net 5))
 (segment (start 33.147 29.337) (end 31.75 27.94) (width 0.254) (layer F.Cu) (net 5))
 (segment (start 33.655 32.258) (end 33.655 30.48) (width 0.254) (layer B.Cu) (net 4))
 (segment (start 30.48 29.21) (end 29.21 27.94) (width 0.254) (layer B.Cu) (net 4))
 (segment (start 32.385 29.21) (end 30.48 29.21) (width 0.254) (layer B.Cu) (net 4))
 (segment (start 33.655 30.48) (end 32.385 29.21) (width 0.254) (layer B.Cu) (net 4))
 (segment (start 35.82416 32.86) (end 35.82416 30.61716) (width 0.254) (layer F.Cu) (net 4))
 (segment (start 35.82416 30.61716) (end 35.687 30.48) (width 0.254) (layer F.Cu) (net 4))
 (segment (start 29.21 27.94) (end 31.242 29.972) (width 0.254) (layer F.Cu) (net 4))
 (segment (start 34.544 29.972) (end 31.242 29.972) (width 0.254) (layer F.Cu) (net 4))
 (segment (start 35.052 30.48) (end 34.544 29.972) (width 0.254) (layer F.Cu) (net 4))
 (segment (start 35.687 30.48) (end 35.052 30.48) (width 0.254) (layer F.Cu) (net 4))
 (segment (start 43.815 32.258) (end 43.815 30.48) (width 0.254) (layer B.Cu) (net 12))
 (segment (start 44.45 29.845) (end 49.53 29.845) (width 0.254) (layer B.Cu) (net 12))
 (segment (start 43.815 30.48) (end 44.45 29.845) (width 0.254) (layer B.Cu) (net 12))
 (segment (start 49.53 34.544) (end 49.53 30.607) (width 0.254) (layer F.Cu) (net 12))
 (via (at 49.53 30.607) (size 0.889) (layers F.Cu B.Cu) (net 12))
 (segment (start 49.022 35.052) (end 49.53 34.544) (width 0.254) (layer F.Cu) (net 12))
 (segment (start 41.02608 34.93008) (end 41.148 35.052) (width 0.254) (layer F.Cu) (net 12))
 (segment (start 41.148 35.052) (end 41.275 35.052) (width 0.254) (layer F.Cu) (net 12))
 (segment (start 41.02608 32.86) (end 41.02608 34.93008) (width 0.254) (layer F.Cu) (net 12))
 (segment (start 41.275 35.052) (end 49.022 35.052) (width 0.254) (layer F.Cu) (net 12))
 (segment (start 49.53 30.607) (end 49.53 29.845) (width 0.254) (layer B.Cu) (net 12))
 (segment (start 49.53 29.845) (end 49.53 27.94) (width 0.254) (layer B.Cu) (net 12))
 (segment (start 45.085 32.258) (end 45.085 34.29) (width 0.254) (layer B.Cu) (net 13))
 (segment (start 52.07 34.29) (end 52.07 27.94) (width 0.254) (layer B.Cu) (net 13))
 (segment (start 51.435 34.925) (end 52.07 34.29) (width 0.254) (layer B.Cu) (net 13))
 (segment (start 45.72 34.925) (end 51.435 34.925) (width 0.254) (layer B.Cu) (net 13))
 (segment (start 45.085 34.29) (end 45.72 34.925) (width 0.254) (layer B.Cu) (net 13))
 (segment (start 45.212 30.48) (end 46.355 29.337) (width 0.254) (layer F.Cu) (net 13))
 (segment (start 50.673 29.337) (end 52.07 27.94) (width 0.254) (layer F.Cu) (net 13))
 (segment (start 46.355 29.337) (end 50.673 29.337) (width 0.254) (layer F.Cu) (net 13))
 (segment (start 41.67378 30.71622) (end 41.91 30.48) (width 0.254) (layer F.Cu) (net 13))
 (segment (start 41.91 30.48) (end 45.212 30.48) (width 0.254) (layer F.Cu) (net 13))
 (segment (start 41.67378 31.96082) (end 41.67378 30.71622) (width 0.254) (layer F.Cu) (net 13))
 (segment (start 46.355 32.258) (end 50.292 32.258) (width 0.254) (layer B.Cu) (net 14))
 (segment (start 50.8 31.75) (end 54.61 27.94) (width 0.254) (layer F.Cu) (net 14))
 (via (at 50.8 31.75) (size 0.889) (layers F.Cu B.Cu) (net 14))
 (segment (start 50.292 32.258) (end 50.8 31.75) (width 0.254) (layer B.Cu) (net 14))
 (segment (start 54.61 27.94) (end 52.705 29.845) (width 0.254) (layer F.Cu) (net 14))
 (segment (start 42.32402 31.46298) (end 42.799 30.988) (width 0.254) (layer F.Cu) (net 14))
 (segment (start 42.799 30.988) (end 45.339 30.988) (width 0.254) (layer F.Cu) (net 14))
 (segment (start 45.339 30.988) (end 46.482 29.845) (width 0.254) (layer F.Cu) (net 14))
 (segment (start 42.32402 31.46298) (end 42.32402 32.86) (width 0.254) (layer F.Cu) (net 14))
 (segment (start 46.482 29.845) (end 52.705 29.845) (width 0.254) (layer F.Cu) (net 14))
 (segment (start 42.545 32.258) (end 42.545 30.48) (width 0.254) (layer B.Cu) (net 11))
 (segment (start 45.72 29.21) (end 46.99 27.94) (width 0.254) (layer B.Cu) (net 11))
 (segment (start 43.815 29.21) (end 45.72 29.21) (width 0.254) (layer B.Cu) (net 11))
 (segment (start 42.545 30.48) (end 43.815 29.21) (width 0.254) (layer B.Cu) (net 11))
 (segment (start 40.37584 32.86) (end 40.37584 30.61716) (width 0.254) (layer F.Cu) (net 11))
 (segment (start 40.37584 30.61716) (end 40.513 30.48) (width 0.254) (layer F.Cu) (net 11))
 (segment (start 40.513 30.48) (end 41.148 30.48) (width 0.254) (layer F.Cu) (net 11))
 (segment (start 41.148 30.48) (end 41.656002 29.971998) (width 0.254) (layer F.Cu) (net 11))
 (segment (start 41.656002 29.971998) (end 44.958002 29.971998) (width 0.254) (layer F.Cu) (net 11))
 (segment (start 44.958002 29.971998) (end 46.99 27.94) (width 0.254) (layer F.Cu) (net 11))
 (segment (start 29.845 32.258) (end 25.908 32.258) (width 0.254) (layer B.Cu) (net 1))
 (segment (start 25.4 31.75) (end 21.59 27.94) (width 0.254) (layer F.Cu) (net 1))
 (via (at 25.4 31.75) (size 0.889) (layers F.Cu B.Cu) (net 1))
 (segment (start 25.908 32.258) (end 25.4 31.75) (width 0.254) (layer B.Cu) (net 1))
 (segment (start 33.87598 32.86) (end 33.87598 31.46298) (width 0.254) (layer F.Cu) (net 1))
 (segment (start 29.464 29.718) (end 23.368 29.718) (width 0.254) (layer F.Cu) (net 1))
 (segment (start 30.734 30.988) (end 29.464 29.718) (width 0.254) (layer F.Cu) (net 1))
 (segment (start 33.401 30.988) (end 30.734 30.988) (width 0.254) (layer F.Cu) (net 1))
 (segment (start 33.87598 31.46298) (end 33.401 30.988) (width 0.254) (layer F.Cu) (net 1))
 (segment (start 23.368 29.718) (end 21.59 27.94) (width 0.254) (layer F.Cu) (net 1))
 (segment (start 41.275 32.258) (end 41.275 30.48) (width 0.254) (layer B.Cu) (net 10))
 (segment (start 42.545 29.845) (end 44.45 27.94) (width 0.254) (layer B.Cu) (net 10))
 (segment (start 41.91 29.845) (end 42.545 29.845) (width 0.254) (layer B.Cu) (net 10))
 (segment (start 41.275 30.48) (end 41.91 29.845) (width 0.254) (layer B.Cu) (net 10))
 (segment (start 39.7256 32.86) (end 39.7256 30.3784) (width 0.254) (layer F.Cu) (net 10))
 (segment (start 43.053 29.337) (end 44.45 27.94) (width 0.254) (layer F.Cu) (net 10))
 (segment (start 39.7256 30.3784) (end 40.259 29.845) (width 0.254) (layer F.Cu) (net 10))
 (segment (start 40.259 29.845) (end 40.894 29.845) (width 0.254) (layer F.Cu) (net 10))
 (segment (start 40.894 29.845) (end 41.402 29.337) (width 0.254) (layer F.Cu) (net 10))
 (segment (start 41.402 29.337) (end 43.053 29.337) (width 0.254) (layer F.Cu) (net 10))
 (segment (start 29.845 38.862) (end 25.908 38.862) (width 0.254) (layer B.Cu) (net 28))
 (segment (start 25.4 39.37) (end 21.59 43.18) (width 0.254) (layer F.Cu) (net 28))
 (via (at 25.4 39.37) (size 0.889) (layers F.Cu B.Cu) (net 28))
 (segment (start 25.908 38.862) (end 25.4 39.37) (width 0.254) (layer B.Cu) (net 28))
 (segment (start 33.87598 38.26) (end 33.87598 39.65702) (width 0.254) (layer F.Cu) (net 28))
 (segment (start 29.337 41.275) (end 23.495 41.275) (width 0.254) (layer F.Cu) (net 28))
 (segment (start 30.48 40.132) (end 29.337 41.275) (width 0.254) (layer F.Cu) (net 28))
 (segment (start 33.401 40.132) (end 30.48 40.132) (width 0.254) (layer F.Cu) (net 28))
 (segment (start 33.87598 39.65702) (end 33.401 40.132) (width 0.254) (layer F.Cu) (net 28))
 (segment (start 23.495 41.275) (end 21.59 43.18) (width 0.254) (layer F.Cu) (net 28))
 (segment (start 31.115 38.862) (end 31.115 36.83) (width 0.254) (layer B.Cu) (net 27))
 (segment (start 24.13 36.83) (end 24.13 43.18) (width 0.254) (layer B.Cu) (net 27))
 (segment (start 24.765 36.195) (end 24.13 36.83) (width 0.254) (layer B.Cu) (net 27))
 (segment (start 30.48 36.195) (end 24.765 36.195) (width 0.254) (layer B.Cu) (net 27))
 (segment (start 31.115 36.83) (end 30.48 36.195) (width 0.254) (layer B.Cu) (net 27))
 (segment (start 30.861 40.64) (end 29.718 41.783) (width 0.254) (layer F.Cu) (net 27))
 (segment (start 25.527 41.783) (end 24.13 43.18) (width 0.254) (layer F.Cu) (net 27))
 (segment (start 29.718 41.783) (end 25.527 41.783) (width 0.254) (layer F.Cu) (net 27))
 (segment (start 34.52622 39.15918) (end 34.52622 40.40378) (width 0.254) (layer F.Cu) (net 27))
 (segment (start 34.29 40.64) (end 30.861 40.64) (width 0.254) (layer F.Cu) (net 27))
 (segment (start 34.52622 40.40378) (end 34.29 40.64) (width 0.254) (layer F.Cu) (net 27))
 (segment (start 32.385 38.862) (end 32.385 40.64) (width 0.254) (layer B.Cu) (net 26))
 (segment (start 31.75 41.275) (end 26.67 41.275) (width 0.254) (layer B.Cu) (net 26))
 (segment (start 32.385 40.64) (end 31.75 41.275) (width 0.254) (layer B.Cu) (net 26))
 (segment (start 26.67 43.18) (end 26.67 41.275) (width 0.254) (layer B.Cu) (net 26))
 (segment (start 26.67 41.275) (end 26.67 40.513) (width 0.254) (layer B.Cu) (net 26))
 (segment (start 26.67 40.513) (end 26.67 36.576) (width 0.254) (layer F.Cu) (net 26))
 (via (at 26.67 40.513) (size 0.889) (layers F.Cu B.Cu) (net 26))
 (segment (start 27.178 36.068) (end 26.67 36.576) (width 0.254) (layer F.Cu) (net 26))
 (segment (start 34.925 36.068) (end 27.178 36.068) (width 0.254) (layer F.Cu) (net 26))
 (segment (start 35.17392 38.26) (end 35.17392 36.18992) (width 0.254) (layer F.Cu) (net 26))
 (segment (start 35.052 36.068) (end 34.925 36.068) (width 0.254) (layer F.Cu) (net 26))
 (segment (start 35.17392 36.18992) (end 35.052 36.068) (width 0.254) (layer F.Cu) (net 26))
 (segment (start 33.655 38.862) (end 33.655 40.64) (width 0.254) (layer B.Cu) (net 25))
 (segment (start 30.48 41.91) (end 29.21 43.18) (width 0.254) (layer B.Cu) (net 25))
 (segment (start 32.385 41.91) (end 30.48 41.91) (width 0.254) (layer B.Cu) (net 25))
 (segment (start 33.655 40.64) (end 32.385 41.91) (width 0.254) (layer B.Cu) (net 25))
 (segment (start 35.82416 38.26) (end 35.82416 40.50284) (width 0.254) (layer F.Cu) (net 25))
 (segment (start 31.241998 41.148002) (end 29.21 43.18) (width 0.254) (layer F.Cu) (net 25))
 (segment (start 34.543998 41.148002) (end 31.241998 41.148002) (width 0.254) (layer F.Cu) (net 25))
 (segment (start 35.052 40.64) (end 34.543998 41.148002) (width 0.254) (layer F.Cu) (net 25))
 (segment (start 35.687 40.64) (end 35.052 40.64) (width 0.254) (layer F.Cu) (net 25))
 (segment (start 35.82416 40.50284) (end 35.687 40.64) (width 0.254) (layer F.Cu) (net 25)))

